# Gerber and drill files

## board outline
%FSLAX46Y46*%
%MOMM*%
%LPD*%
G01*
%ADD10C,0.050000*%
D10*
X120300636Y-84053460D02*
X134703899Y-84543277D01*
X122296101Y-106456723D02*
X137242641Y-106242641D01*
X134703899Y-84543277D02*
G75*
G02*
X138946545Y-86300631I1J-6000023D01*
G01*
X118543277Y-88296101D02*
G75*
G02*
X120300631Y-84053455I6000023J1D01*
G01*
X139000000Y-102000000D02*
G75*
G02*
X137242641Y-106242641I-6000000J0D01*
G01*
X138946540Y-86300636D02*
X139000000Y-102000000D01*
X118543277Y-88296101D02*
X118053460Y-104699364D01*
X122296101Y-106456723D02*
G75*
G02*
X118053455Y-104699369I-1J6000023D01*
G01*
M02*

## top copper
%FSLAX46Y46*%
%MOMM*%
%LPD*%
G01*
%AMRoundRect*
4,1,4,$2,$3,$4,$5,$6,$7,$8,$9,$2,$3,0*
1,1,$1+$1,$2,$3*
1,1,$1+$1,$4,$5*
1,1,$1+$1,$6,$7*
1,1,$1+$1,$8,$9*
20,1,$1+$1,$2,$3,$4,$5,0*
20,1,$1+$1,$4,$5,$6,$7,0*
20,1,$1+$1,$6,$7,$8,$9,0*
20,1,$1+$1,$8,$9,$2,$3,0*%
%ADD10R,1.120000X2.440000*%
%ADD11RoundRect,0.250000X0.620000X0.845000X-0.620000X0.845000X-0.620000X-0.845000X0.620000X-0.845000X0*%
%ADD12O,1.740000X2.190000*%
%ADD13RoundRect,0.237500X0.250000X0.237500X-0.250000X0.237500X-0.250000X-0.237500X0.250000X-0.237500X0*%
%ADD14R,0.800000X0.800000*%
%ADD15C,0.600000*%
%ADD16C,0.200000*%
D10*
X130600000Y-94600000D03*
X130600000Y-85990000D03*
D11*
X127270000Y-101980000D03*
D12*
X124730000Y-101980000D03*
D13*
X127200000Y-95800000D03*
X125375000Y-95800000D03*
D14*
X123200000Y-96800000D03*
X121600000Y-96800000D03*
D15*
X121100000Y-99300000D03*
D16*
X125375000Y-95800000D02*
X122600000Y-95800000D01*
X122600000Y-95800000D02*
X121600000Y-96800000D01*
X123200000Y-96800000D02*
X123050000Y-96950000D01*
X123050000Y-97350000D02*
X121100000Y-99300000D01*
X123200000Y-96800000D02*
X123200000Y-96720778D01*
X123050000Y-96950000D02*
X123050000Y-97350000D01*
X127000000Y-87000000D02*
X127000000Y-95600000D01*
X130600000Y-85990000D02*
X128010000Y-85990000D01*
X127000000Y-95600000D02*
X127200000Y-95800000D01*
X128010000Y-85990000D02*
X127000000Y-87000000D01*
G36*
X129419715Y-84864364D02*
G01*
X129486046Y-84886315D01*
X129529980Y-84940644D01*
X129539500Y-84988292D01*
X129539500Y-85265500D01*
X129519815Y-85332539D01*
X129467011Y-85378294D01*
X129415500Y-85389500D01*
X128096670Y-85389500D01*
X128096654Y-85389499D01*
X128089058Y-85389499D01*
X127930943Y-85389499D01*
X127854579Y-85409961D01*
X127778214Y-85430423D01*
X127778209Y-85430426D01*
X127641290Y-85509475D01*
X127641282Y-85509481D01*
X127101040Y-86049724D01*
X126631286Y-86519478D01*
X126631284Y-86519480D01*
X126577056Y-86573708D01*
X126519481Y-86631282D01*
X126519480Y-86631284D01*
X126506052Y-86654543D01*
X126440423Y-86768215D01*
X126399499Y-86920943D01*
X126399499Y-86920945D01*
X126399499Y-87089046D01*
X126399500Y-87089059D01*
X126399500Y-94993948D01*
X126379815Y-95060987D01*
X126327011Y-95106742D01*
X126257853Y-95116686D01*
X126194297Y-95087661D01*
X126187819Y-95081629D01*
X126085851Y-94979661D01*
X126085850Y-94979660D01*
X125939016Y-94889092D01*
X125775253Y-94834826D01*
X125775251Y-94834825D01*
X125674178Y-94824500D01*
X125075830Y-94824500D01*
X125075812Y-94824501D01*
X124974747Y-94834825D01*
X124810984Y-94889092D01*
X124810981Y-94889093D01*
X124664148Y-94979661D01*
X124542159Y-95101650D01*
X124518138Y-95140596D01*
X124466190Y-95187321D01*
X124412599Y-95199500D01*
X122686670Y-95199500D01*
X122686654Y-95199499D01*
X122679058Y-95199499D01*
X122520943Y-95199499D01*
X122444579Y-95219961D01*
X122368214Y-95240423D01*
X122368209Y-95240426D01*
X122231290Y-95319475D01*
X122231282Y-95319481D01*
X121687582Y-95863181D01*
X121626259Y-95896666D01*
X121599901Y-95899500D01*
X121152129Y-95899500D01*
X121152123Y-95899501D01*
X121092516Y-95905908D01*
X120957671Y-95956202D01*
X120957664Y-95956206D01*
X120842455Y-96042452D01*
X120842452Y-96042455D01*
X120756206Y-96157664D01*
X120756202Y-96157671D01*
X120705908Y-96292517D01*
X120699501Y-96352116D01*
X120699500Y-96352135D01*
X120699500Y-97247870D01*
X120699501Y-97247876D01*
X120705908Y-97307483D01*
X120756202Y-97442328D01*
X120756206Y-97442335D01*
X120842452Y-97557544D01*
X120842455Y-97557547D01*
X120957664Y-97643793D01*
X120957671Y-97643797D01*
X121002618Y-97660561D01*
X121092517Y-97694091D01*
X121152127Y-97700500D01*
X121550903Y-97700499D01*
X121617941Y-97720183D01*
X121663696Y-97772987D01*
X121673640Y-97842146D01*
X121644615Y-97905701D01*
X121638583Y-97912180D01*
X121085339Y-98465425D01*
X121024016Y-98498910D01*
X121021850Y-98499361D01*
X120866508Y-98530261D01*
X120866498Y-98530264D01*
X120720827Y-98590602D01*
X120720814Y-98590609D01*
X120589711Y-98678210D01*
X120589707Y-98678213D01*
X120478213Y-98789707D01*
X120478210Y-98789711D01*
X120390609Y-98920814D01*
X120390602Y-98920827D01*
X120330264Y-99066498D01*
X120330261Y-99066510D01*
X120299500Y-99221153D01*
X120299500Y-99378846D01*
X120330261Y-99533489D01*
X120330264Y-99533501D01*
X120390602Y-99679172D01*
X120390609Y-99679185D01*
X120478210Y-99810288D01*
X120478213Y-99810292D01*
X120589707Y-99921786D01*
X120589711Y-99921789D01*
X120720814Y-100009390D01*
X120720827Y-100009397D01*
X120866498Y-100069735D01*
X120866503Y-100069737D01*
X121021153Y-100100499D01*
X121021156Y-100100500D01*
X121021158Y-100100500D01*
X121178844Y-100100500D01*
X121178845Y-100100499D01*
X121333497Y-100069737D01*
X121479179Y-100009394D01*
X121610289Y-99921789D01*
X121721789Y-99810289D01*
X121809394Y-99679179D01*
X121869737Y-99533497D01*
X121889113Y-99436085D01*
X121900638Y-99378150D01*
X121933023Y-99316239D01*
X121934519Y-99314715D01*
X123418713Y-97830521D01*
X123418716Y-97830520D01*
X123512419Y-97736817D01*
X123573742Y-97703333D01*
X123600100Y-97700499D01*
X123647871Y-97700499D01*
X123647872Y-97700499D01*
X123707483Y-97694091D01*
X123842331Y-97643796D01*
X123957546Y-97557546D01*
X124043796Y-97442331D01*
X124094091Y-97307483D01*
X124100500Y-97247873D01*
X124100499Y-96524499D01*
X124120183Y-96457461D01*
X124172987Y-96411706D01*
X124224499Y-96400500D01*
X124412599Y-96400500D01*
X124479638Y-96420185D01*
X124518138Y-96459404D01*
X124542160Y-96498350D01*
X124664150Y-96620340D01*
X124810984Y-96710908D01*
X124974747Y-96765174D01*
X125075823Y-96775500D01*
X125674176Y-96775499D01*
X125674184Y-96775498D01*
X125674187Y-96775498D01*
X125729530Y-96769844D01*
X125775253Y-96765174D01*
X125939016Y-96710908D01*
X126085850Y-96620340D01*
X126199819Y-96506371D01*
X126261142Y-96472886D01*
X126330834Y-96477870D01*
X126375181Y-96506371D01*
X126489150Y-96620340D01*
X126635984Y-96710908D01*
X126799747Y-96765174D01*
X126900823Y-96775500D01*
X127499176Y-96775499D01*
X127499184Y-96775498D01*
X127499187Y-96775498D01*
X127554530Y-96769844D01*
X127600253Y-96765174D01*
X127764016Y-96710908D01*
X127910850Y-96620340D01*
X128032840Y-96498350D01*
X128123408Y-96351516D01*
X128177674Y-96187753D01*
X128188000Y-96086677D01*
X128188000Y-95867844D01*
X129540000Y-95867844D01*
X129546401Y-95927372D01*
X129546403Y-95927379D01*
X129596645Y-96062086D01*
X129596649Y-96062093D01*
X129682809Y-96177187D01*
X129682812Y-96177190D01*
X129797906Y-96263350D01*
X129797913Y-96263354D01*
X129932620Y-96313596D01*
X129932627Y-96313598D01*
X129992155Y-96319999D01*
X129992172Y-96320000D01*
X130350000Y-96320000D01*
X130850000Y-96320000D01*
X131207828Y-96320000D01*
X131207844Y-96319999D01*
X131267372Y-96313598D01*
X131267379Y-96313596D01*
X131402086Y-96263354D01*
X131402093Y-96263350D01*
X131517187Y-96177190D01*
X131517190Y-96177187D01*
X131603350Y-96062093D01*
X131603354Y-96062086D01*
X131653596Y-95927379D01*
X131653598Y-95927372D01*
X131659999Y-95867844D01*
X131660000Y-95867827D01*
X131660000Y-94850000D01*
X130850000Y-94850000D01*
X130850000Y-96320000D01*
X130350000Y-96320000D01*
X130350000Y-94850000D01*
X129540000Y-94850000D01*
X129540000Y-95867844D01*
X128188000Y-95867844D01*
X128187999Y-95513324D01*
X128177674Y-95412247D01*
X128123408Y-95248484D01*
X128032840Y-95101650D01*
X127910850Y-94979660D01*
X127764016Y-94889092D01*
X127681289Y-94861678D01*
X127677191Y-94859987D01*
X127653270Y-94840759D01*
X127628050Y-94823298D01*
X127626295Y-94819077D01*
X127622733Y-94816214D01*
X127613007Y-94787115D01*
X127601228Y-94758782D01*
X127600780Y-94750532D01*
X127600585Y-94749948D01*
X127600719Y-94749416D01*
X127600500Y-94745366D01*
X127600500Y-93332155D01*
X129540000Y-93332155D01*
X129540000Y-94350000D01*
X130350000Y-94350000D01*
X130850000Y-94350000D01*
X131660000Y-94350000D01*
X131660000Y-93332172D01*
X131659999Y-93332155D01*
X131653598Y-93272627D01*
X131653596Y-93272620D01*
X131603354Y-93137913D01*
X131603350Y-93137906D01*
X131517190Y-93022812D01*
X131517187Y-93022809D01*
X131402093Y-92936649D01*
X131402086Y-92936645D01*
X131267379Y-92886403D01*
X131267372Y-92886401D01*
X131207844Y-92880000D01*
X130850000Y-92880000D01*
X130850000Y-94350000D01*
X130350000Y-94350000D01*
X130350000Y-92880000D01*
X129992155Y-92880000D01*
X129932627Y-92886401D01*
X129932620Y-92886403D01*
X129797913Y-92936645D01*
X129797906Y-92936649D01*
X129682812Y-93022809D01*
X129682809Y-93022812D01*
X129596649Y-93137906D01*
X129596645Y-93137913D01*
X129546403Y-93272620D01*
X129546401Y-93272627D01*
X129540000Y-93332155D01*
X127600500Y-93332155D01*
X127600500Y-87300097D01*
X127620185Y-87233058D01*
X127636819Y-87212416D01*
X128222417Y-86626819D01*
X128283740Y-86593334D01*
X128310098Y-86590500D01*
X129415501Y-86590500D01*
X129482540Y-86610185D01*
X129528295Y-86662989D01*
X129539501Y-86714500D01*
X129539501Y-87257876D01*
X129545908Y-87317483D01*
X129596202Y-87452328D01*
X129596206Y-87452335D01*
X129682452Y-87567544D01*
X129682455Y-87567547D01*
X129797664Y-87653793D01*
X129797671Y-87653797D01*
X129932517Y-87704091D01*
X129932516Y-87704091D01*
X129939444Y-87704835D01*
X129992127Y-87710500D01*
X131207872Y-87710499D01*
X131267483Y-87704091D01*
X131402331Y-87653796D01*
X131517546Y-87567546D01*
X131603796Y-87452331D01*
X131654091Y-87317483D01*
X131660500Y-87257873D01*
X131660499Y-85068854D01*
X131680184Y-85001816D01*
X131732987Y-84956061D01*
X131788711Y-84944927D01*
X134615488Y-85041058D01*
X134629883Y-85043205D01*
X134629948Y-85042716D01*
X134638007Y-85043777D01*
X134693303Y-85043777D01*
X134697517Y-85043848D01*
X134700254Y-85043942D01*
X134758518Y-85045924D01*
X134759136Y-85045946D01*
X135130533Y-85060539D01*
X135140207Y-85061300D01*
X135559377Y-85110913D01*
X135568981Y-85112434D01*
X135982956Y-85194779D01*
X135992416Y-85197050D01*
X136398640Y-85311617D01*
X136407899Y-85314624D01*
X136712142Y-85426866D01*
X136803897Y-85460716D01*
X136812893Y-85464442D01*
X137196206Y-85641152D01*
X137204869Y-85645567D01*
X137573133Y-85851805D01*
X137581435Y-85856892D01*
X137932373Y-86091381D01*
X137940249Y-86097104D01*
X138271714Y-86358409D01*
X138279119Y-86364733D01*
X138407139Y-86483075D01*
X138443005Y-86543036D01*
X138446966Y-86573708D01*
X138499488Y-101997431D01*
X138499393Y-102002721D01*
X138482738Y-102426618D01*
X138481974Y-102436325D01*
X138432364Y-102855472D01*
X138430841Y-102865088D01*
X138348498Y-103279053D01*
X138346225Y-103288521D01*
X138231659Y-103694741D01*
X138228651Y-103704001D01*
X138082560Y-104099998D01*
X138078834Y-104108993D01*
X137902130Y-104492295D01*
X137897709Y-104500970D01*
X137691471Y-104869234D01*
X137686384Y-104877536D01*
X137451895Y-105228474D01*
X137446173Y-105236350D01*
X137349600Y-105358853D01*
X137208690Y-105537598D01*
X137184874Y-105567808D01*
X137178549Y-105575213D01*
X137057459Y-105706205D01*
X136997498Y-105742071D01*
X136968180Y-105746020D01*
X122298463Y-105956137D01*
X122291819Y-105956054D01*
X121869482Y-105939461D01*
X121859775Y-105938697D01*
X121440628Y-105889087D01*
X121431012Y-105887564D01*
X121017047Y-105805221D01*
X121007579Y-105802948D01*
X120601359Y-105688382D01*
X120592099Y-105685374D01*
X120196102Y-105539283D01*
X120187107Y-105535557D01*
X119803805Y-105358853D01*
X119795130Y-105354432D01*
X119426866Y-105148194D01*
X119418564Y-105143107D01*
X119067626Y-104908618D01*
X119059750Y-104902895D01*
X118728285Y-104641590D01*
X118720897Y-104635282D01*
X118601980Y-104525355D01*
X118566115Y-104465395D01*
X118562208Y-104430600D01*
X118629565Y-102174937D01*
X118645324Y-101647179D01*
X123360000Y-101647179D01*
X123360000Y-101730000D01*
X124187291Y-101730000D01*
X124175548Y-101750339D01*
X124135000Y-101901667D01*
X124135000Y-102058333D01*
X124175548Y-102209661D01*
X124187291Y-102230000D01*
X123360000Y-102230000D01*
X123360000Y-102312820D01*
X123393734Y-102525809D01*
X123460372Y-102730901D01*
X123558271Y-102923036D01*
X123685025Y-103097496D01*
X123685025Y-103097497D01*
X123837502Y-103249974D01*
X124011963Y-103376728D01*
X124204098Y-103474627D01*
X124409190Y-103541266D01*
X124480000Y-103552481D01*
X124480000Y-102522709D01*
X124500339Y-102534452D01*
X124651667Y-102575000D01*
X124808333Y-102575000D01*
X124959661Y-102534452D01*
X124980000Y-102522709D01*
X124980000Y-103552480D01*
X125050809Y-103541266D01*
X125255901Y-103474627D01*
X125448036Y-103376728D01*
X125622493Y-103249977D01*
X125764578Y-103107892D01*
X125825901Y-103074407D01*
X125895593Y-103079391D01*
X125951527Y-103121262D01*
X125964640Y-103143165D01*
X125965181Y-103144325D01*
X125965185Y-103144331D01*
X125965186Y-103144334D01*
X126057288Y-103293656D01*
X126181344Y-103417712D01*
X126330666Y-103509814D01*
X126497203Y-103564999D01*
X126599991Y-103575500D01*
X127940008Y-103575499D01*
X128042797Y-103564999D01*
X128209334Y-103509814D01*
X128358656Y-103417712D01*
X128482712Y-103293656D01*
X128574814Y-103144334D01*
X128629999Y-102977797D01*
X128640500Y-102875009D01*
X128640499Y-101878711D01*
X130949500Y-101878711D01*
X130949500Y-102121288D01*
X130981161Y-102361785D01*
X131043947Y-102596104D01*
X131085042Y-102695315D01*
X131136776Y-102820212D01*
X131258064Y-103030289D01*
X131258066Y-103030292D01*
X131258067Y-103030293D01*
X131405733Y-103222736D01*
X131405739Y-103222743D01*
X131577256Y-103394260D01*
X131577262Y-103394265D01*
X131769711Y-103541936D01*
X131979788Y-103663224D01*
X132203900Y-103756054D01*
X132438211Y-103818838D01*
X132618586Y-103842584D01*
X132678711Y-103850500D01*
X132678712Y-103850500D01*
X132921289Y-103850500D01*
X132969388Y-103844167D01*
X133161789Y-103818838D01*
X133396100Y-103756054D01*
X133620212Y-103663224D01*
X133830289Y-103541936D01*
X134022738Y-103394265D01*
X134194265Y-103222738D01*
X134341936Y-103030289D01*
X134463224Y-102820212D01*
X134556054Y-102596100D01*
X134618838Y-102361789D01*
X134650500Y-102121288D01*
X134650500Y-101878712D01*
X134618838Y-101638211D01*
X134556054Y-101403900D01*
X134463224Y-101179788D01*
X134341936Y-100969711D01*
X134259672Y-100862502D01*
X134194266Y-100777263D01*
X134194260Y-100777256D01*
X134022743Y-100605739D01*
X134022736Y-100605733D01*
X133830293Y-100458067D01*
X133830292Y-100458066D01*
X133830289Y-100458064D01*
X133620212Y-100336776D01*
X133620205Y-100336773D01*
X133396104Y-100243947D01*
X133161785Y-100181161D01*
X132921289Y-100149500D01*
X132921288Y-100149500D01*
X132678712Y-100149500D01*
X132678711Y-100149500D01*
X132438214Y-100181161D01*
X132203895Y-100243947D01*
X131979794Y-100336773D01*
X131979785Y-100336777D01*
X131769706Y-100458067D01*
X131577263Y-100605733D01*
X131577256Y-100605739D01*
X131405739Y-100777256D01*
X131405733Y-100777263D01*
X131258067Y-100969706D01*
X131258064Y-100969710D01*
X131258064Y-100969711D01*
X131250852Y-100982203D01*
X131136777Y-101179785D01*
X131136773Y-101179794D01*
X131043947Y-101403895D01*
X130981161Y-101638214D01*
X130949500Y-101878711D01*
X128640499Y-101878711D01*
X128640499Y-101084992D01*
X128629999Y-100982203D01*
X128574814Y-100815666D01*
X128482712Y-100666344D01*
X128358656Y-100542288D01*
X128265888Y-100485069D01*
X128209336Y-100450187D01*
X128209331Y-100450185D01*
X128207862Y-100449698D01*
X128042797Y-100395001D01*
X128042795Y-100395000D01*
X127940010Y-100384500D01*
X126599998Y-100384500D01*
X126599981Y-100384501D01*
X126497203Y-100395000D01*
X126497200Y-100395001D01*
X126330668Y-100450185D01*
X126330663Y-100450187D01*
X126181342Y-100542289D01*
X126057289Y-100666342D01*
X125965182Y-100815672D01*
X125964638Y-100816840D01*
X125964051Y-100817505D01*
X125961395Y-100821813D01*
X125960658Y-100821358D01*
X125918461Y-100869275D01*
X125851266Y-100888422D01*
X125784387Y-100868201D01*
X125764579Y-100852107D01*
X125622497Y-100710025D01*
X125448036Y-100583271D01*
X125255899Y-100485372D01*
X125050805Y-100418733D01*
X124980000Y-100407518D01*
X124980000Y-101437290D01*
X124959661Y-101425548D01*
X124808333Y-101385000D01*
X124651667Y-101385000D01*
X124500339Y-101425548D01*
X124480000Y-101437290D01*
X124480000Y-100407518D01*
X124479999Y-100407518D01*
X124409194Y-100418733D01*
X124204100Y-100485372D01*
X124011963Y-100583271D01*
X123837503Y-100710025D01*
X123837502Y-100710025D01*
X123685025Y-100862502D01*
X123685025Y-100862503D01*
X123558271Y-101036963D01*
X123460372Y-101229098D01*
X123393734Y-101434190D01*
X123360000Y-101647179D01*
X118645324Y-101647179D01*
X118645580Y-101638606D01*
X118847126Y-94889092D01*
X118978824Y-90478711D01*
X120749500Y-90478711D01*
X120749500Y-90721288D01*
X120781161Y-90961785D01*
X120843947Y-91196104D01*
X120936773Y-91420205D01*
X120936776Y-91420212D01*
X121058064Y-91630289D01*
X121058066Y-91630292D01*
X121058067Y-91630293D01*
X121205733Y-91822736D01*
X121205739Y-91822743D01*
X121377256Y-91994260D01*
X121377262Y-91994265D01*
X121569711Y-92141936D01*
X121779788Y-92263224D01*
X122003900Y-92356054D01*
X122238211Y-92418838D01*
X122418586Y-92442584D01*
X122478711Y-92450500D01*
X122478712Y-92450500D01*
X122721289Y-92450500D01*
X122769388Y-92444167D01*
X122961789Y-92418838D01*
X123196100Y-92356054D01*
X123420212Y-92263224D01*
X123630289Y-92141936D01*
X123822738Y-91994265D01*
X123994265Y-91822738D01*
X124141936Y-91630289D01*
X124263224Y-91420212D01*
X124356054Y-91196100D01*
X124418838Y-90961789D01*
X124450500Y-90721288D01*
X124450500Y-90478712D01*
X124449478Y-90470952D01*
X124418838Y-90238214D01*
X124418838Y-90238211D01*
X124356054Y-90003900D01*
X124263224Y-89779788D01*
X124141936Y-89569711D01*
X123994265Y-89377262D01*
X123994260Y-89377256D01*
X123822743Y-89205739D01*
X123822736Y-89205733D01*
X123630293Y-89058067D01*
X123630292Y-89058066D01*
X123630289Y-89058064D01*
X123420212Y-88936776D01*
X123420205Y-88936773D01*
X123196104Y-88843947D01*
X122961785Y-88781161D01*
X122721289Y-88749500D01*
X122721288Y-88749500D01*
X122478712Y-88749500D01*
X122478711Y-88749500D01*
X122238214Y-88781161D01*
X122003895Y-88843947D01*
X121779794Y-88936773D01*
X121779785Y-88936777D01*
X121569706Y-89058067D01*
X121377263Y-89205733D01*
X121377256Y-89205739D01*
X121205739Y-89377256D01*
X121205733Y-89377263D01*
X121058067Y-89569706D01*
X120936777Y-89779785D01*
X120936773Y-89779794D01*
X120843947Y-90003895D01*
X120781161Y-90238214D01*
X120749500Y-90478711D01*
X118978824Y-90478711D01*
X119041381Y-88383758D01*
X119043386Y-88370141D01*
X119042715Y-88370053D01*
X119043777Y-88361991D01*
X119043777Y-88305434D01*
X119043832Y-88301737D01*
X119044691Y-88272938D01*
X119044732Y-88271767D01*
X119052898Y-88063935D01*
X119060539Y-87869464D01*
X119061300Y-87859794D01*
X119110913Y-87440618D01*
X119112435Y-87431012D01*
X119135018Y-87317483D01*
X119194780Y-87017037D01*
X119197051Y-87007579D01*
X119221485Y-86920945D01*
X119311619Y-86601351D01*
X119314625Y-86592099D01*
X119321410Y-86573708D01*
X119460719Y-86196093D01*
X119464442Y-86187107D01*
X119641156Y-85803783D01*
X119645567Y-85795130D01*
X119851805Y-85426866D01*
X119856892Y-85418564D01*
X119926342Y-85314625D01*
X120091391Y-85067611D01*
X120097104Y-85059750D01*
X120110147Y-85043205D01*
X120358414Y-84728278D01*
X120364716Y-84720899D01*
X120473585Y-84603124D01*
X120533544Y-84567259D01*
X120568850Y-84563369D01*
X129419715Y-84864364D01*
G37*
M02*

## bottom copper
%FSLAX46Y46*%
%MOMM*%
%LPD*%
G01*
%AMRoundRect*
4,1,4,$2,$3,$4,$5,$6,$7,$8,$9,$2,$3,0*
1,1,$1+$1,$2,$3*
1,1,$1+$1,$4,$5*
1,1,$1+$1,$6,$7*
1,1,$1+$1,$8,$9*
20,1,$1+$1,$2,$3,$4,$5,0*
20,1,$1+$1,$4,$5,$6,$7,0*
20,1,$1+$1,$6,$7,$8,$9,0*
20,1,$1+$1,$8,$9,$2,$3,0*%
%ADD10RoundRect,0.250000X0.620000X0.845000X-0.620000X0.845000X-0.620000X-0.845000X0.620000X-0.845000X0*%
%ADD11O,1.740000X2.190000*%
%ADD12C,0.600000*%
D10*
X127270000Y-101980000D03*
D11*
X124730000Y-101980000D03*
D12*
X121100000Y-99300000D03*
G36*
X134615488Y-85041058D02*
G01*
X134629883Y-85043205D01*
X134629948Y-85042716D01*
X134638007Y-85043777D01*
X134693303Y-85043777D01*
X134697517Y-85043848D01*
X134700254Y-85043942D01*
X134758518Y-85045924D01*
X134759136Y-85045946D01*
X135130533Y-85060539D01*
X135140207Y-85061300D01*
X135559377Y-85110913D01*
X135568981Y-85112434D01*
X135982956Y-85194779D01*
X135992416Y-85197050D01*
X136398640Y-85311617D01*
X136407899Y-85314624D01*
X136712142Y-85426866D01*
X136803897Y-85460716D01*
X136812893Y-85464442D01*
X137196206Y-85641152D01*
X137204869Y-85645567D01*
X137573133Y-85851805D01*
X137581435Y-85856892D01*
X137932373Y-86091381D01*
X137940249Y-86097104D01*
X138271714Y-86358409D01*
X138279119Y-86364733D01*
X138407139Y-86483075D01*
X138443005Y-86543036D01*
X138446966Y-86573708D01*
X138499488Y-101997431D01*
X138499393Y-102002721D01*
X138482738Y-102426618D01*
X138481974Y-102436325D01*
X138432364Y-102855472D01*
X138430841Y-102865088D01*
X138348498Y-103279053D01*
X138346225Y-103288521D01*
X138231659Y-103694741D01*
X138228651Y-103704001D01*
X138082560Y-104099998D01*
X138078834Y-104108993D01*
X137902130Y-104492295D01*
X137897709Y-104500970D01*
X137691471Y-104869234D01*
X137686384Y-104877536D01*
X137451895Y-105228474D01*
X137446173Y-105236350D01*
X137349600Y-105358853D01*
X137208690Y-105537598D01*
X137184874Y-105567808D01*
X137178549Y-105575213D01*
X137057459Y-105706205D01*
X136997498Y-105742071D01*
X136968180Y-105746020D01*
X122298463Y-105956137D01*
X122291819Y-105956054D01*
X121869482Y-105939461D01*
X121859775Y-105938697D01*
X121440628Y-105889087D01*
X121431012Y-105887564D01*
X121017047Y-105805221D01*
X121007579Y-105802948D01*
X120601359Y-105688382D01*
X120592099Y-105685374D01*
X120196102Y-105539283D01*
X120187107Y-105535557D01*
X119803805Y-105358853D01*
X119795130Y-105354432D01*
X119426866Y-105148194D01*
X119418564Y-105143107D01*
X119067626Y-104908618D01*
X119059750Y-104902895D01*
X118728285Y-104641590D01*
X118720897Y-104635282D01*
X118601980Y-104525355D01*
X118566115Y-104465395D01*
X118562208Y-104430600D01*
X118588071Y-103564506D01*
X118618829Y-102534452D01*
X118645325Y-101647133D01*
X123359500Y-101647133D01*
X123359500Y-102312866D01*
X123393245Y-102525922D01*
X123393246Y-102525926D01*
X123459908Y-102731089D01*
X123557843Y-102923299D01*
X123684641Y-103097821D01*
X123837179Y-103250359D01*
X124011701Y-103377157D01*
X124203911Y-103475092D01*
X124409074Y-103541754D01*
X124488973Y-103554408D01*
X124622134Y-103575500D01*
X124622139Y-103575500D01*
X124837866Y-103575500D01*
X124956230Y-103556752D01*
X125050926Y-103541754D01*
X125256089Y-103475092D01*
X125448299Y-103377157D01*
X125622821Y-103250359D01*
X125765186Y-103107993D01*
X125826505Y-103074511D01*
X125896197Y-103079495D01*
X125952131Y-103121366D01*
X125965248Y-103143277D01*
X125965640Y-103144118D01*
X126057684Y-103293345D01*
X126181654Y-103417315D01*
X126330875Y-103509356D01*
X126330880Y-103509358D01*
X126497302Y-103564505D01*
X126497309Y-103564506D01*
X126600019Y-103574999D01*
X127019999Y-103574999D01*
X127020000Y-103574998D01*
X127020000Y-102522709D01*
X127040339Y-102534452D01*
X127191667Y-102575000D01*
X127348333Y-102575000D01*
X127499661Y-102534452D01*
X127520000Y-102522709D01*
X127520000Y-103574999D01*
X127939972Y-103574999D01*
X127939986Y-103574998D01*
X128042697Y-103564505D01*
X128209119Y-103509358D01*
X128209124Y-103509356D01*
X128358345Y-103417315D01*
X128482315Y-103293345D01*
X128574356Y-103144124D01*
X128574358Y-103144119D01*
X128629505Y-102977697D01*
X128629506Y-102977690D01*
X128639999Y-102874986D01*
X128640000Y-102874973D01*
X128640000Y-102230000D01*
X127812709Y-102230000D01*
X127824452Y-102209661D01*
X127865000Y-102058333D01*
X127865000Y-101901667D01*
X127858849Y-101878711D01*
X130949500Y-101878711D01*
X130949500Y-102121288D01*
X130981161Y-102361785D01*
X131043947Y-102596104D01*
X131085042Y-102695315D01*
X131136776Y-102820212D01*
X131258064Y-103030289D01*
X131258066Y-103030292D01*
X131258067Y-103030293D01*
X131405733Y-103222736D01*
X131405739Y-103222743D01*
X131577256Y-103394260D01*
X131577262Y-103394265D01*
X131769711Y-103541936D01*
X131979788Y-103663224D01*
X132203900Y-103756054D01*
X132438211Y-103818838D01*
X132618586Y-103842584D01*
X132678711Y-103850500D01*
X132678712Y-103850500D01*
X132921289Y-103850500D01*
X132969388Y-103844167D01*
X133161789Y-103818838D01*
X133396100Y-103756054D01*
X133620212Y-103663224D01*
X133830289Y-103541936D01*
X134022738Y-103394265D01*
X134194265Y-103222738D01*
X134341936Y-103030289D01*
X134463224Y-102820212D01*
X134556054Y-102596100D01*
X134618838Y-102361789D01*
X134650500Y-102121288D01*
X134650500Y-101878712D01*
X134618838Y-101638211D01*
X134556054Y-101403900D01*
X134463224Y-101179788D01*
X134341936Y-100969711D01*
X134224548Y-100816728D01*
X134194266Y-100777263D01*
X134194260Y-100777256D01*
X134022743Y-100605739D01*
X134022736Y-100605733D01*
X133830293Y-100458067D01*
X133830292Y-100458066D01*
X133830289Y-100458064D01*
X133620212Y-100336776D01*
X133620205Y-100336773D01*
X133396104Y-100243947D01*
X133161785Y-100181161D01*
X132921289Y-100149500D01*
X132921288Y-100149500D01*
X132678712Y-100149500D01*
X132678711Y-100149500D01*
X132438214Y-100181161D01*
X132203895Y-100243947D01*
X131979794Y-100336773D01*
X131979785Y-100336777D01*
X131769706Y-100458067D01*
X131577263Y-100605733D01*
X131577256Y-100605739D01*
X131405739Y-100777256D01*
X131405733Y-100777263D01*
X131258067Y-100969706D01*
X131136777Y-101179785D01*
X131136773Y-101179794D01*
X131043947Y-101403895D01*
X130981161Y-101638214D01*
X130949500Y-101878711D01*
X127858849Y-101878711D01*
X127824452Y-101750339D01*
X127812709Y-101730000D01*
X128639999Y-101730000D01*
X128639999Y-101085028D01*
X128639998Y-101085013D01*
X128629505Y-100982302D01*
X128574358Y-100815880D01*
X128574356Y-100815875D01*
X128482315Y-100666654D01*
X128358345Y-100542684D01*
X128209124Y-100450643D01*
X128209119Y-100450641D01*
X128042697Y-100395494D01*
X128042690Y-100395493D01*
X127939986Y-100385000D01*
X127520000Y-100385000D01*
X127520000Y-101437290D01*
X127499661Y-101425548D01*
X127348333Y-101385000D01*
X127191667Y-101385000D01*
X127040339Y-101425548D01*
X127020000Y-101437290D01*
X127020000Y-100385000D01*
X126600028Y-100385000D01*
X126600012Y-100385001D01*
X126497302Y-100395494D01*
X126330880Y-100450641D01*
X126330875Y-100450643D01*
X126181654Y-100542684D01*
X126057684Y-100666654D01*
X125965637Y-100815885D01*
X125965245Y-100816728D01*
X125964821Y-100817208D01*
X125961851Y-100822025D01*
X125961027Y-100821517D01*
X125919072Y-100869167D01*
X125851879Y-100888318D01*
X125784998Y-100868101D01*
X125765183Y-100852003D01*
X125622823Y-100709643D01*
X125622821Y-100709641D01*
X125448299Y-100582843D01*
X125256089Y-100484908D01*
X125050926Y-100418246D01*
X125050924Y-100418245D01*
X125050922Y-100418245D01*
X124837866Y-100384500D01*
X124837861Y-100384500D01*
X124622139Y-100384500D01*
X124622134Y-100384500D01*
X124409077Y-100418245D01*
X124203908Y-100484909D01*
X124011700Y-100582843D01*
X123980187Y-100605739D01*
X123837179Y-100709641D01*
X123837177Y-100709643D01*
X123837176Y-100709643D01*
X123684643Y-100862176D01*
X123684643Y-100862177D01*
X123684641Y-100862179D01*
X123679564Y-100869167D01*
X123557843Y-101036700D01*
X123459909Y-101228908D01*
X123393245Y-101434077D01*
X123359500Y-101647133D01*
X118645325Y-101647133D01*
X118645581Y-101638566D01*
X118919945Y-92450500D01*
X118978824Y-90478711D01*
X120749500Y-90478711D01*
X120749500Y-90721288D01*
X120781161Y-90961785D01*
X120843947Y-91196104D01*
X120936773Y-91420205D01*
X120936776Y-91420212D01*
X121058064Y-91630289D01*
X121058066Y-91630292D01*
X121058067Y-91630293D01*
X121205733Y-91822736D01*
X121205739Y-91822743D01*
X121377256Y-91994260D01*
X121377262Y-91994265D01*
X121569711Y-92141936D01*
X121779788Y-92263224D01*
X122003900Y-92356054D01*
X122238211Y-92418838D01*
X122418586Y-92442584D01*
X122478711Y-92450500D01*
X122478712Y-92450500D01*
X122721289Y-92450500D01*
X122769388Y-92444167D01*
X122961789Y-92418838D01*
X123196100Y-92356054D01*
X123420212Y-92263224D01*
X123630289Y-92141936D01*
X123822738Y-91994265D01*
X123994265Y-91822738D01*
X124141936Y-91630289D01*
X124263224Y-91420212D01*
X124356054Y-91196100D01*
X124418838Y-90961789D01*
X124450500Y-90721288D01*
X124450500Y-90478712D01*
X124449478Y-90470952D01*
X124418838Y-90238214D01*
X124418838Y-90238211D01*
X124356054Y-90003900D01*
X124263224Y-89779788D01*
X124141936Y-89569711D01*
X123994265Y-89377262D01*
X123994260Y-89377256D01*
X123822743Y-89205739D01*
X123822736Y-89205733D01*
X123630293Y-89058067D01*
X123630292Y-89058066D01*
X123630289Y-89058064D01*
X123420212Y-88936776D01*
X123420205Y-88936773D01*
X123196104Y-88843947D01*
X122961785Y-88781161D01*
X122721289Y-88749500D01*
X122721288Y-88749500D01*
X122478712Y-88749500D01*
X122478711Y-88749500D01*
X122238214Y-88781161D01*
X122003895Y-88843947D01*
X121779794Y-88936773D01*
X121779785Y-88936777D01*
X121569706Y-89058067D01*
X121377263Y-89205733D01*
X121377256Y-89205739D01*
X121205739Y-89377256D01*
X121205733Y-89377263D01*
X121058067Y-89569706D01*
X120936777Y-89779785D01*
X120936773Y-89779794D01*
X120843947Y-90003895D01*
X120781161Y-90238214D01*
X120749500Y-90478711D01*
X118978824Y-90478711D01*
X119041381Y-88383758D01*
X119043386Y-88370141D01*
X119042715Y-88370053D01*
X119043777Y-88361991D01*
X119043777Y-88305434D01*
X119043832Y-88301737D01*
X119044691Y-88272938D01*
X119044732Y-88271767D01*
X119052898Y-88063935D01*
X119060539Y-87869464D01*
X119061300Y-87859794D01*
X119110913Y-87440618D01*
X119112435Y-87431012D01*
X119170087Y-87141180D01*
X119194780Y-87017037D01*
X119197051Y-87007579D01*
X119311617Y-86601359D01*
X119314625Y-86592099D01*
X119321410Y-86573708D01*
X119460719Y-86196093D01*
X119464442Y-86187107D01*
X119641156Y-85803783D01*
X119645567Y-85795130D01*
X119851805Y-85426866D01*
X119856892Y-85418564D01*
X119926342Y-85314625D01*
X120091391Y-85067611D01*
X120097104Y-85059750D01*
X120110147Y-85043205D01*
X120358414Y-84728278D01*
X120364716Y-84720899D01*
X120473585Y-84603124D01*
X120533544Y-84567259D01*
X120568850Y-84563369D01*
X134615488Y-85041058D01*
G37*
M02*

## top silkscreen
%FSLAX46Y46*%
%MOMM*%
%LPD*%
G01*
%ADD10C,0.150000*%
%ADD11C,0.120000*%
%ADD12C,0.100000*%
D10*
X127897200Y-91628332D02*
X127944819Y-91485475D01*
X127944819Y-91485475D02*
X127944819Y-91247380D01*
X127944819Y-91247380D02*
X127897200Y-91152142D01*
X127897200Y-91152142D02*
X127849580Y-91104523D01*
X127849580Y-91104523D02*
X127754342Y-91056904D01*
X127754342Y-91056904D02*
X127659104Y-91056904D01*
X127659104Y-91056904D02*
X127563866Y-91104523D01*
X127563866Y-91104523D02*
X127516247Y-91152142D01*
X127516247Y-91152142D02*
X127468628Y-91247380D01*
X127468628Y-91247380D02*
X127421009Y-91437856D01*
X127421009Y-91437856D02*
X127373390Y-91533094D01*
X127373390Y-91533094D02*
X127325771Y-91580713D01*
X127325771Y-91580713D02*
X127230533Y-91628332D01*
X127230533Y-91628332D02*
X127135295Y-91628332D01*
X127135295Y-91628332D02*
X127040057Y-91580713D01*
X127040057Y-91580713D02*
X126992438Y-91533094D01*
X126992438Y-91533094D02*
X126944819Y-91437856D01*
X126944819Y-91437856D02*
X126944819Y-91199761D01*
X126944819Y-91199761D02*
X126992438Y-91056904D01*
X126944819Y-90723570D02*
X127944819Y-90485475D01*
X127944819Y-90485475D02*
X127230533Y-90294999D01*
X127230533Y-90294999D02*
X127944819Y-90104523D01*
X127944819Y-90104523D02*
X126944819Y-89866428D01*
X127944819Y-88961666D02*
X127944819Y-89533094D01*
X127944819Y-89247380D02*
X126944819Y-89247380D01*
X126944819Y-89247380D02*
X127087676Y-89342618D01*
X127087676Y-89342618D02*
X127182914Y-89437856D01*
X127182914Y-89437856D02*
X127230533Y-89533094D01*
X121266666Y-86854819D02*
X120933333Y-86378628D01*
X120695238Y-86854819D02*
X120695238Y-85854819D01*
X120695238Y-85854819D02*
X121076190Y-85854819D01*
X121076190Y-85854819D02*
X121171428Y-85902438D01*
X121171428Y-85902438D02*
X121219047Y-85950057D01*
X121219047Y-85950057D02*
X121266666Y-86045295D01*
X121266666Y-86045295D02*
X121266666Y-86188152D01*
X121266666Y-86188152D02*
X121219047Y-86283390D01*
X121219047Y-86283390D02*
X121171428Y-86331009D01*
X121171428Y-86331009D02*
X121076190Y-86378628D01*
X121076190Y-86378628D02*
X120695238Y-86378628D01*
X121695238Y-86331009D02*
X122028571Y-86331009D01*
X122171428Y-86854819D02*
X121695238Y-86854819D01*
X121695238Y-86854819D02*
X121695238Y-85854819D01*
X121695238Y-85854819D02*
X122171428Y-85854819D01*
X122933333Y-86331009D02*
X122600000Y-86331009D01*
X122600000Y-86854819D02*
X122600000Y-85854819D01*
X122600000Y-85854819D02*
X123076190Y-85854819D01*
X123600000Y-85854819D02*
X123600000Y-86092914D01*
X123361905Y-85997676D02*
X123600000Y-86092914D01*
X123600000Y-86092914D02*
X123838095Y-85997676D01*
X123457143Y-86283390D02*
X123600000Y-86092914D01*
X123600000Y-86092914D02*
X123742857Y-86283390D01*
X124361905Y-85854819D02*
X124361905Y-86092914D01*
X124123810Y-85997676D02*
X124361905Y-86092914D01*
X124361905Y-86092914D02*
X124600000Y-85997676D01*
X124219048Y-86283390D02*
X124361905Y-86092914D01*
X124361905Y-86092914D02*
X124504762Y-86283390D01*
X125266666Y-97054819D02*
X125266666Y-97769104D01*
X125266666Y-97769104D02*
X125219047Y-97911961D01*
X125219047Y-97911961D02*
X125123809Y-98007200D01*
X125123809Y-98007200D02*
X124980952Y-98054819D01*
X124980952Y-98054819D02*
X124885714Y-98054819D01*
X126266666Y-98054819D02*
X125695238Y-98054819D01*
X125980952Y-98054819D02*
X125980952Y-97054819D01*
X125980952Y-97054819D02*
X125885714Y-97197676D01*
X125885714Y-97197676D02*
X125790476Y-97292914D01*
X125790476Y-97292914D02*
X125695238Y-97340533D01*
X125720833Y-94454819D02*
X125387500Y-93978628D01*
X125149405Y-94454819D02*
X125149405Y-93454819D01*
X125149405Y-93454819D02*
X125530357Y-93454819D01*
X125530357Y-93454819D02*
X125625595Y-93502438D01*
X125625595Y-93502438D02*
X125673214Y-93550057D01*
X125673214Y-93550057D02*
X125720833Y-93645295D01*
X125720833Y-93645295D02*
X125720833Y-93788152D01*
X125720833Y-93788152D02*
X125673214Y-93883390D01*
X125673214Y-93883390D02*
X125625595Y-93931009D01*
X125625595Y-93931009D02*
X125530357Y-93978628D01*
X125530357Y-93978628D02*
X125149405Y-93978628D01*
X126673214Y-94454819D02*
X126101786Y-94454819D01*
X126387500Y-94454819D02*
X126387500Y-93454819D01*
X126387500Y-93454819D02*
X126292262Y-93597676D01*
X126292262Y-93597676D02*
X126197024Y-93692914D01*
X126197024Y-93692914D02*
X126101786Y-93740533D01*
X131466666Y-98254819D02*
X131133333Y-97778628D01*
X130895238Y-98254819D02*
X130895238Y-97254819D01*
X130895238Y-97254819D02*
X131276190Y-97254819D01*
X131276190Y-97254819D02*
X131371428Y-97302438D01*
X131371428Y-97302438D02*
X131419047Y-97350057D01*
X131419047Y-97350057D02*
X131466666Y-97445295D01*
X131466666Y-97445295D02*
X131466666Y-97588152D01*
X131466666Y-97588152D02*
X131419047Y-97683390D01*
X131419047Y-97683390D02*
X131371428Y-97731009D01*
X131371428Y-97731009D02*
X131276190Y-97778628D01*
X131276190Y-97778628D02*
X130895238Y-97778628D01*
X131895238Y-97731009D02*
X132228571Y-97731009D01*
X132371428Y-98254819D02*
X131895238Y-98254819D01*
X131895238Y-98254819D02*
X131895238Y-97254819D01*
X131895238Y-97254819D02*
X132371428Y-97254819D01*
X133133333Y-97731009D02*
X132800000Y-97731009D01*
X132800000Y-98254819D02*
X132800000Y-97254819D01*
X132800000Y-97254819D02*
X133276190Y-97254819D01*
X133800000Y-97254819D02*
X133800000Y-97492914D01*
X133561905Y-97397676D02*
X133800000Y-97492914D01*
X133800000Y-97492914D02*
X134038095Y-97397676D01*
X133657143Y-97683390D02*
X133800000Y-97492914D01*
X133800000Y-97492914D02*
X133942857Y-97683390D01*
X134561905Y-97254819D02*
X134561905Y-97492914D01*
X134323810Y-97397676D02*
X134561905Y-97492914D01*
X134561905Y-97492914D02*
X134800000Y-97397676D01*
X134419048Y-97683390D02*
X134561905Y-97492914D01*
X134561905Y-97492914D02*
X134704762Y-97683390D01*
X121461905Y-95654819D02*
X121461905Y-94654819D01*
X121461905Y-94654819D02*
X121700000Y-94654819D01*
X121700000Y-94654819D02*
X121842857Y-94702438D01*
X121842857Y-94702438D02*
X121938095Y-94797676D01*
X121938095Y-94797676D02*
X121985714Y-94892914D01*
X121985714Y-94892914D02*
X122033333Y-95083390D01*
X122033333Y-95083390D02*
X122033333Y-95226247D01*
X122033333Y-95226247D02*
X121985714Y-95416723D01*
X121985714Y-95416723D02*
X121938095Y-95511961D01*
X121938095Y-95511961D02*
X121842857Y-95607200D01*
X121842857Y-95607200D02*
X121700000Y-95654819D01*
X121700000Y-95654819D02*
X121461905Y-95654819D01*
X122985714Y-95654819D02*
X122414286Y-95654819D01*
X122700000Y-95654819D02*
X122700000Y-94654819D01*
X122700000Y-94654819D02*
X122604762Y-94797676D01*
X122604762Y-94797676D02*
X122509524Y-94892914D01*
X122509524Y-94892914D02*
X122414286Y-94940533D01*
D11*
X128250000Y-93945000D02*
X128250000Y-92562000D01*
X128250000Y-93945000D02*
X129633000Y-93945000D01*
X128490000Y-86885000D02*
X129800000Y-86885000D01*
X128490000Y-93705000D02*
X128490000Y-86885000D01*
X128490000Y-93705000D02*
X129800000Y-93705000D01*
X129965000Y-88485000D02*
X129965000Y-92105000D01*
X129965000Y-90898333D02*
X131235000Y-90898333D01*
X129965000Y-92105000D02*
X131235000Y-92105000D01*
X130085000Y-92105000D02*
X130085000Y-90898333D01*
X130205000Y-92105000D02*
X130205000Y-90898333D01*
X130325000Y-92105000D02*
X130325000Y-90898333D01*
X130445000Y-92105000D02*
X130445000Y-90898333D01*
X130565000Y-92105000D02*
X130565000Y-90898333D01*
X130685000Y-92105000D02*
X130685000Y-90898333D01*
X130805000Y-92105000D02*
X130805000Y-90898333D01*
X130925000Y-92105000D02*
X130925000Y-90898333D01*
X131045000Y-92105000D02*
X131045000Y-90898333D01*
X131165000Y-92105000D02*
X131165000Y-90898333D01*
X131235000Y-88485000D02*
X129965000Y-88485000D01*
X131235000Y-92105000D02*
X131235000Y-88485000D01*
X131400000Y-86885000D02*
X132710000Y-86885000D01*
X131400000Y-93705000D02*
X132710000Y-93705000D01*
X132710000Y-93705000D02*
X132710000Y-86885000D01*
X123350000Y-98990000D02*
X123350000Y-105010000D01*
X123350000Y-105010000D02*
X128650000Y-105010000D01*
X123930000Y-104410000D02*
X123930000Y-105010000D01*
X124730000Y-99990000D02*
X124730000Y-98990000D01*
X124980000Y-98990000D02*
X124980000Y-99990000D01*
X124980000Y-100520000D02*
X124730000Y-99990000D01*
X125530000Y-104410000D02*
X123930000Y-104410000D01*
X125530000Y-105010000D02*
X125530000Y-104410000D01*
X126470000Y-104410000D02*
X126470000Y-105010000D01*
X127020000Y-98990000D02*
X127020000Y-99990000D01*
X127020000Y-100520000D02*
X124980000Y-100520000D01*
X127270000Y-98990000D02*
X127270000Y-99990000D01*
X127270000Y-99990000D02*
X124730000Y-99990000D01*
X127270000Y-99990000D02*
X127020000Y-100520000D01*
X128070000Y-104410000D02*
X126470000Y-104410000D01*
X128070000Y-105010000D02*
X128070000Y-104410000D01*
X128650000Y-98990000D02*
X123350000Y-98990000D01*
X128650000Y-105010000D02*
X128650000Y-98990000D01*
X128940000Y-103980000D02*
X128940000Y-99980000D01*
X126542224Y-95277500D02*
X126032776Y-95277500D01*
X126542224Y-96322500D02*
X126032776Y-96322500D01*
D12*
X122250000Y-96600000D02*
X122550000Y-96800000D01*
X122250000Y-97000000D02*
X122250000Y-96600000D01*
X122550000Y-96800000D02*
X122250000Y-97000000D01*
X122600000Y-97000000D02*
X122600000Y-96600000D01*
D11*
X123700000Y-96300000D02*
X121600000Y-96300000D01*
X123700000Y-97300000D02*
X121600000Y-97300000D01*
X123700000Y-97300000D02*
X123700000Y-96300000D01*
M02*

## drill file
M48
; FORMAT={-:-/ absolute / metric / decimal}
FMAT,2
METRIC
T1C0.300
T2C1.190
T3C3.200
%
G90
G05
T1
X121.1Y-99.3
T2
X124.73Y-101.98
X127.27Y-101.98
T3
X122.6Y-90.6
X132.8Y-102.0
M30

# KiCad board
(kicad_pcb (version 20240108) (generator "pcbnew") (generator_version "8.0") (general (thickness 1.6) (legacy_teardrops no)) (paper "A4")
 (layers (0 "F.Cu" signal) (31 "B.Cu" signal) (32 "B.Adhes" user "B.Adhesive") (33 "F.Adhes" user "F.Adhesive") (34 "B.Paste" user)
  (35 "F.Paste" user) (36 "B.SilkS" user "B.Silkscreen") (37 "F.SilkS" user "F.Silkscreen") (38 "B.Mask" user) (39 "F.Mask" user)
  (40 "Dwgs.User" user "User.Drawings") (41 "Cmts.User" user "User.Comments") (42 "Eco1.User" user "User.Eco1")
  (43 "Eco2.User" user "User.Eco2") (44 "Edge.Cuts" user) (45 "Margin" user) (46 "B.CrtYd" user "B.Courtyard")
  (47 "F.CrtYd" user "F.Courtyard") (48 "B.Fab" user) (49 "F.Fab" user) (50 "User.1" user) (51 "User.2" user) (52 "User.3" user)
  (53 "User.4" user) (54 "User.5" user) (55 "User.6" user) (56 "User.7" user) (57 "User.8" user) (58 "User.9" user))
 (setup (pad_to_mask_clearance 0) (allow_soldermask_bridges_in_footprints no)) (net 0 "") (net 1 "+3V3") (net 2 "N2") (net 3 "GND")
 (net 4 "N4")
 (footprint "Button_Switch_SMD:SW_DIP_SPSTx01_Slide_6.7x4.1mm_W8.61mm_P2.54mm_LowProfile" (layer "F.Cu") (at 130.6 90.295 90)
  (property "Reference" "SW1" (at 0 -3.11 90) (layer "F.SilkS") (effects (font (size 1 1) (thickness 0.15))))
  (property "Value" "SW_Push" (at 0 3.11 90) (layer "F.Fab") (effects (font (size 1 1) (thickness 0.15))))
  (fp_line (start -3.65 -2.35) (end -2.267 -2.35) (stroke (width 0.12) (type solid)) (layer "F.SilkS"))
  (fp_line (start -3.65 -2.35) (end -3.65 -0.967) (stroke (width 0.12) (type solid)) (layer "F.SilkS"))
  (fp_line (start 3.41 -2.11) (end 3.41 -0.8) (stroke (width 0.12) (type solid)) (layer "F.SilkS"))
  (fp_line (start -3.41 -2.11) (end 3.41 -2.11) (stroke (width 0.12) (type solid)) (layer "F.SilkS"))
  (fp_line (start -3.41 -2.11) (end -3.41 -0.8) (stroke (width 0.12) (type solid)) (layer "F.SilkS"))
  (fp_line (start 1.81 -0.635) (end -1.81 -0.635) (stroke (width 0.12) (type solid)) (layer "F.SilkS"))
  (fp_line (start -0.603333 -0.635) (end -0.603333 0.635) (stroke (width 0.12) (type solid)) (layer "F.SilkS"))
  (fp_line (start -1.81 -0.635) (end -1.81 0.635) (stroke (width 0.12) (type solid)) (layer "F.SilkS"))
  (fp_line (start -1.81 -0.515) (end -0.603333 -0.515) (stroke (width 0.12) (type solid)) (layer "F.SilkS"))
  (fp_line (start -1.81 -0.395) (end -0.603333 -0.395) (stroke (width 0.12) (type solid)) (layer "F.SilkS"))
  (fp_line (start -1.81 -0.275) (end -0.603333 -0.275) (stroke (width 0.12) (type solid)) (layer "F.SilkS"))
  (fp_line (start -1.81 -0.155) (end -0.603333 -0.155) (stroke (width 0.12) (type solid)) (layer "F.SilkS"))
  (fp_line (start -1.81 -0.035) (end -0.603333 -0.035) (stroke (width 0.12) (type solid)) (layer "F.SilkS"))
  (fp_line (start -1.81 0.085) (end -0.603333 0.085) (stroke (width 0.12) (type solid)) (layer "F.SilkS"))
  (fp_line (start -1.81 0.205) (end -0.603333 0.205) (stroke (width 0.12) (type solid)) (layer "F.SilkS"))
  (fp_line (start -1.81 0.325) (end -0.603333 0.325) (stroke (width 0.12) (type solid)) (layer "F.SilkS"))
  (fp_line (start -1.81 0.445) (end -0.603333 0.445) (stroke (width 0.12) (type solid)) (layer "F.SilkS"))
  (fp_line (start -1.81 0.565) (end -0.603333 0.565) (stroke (width 0.12) (type solid)) (layer "F.SilkS"))
  (fp_line (start 1.81 0.635) (end 1.81 -0.635) (stroke (width 0.12) (type solid)) (layer "F.SilkS"))
  (fp_line (start -1.81 0.635) (end 1.81 0.635) (stroke (width 0.12) (type solid)) (layer "F.SilkS"))
  (fp_line (start 3.41 0.8) (end 3.41 2.11) (stroke (width 0.12) (type solid)) (layer "F.SilkS"))
  (fp_line (start -3.41 0.8) (end -3.41 2.11) (stroke (width 0.12) (type solid)) (layer "F.SilkS"))
  (fp_line (start -3.41 2.11) (end 3.41 2.11) (stroke (width 0.12) (type solid)) (layer "F.SilkS"))
  (pad "1" smd rect (at -4.305 0 90) (size 2.44 1.12) (layers "F.Cu" "F.Paste" "F.Mask") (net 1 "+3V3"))
  (pad "2" smd rect (at 4.305 0 90) (size 2.44 1.12) (layers "F.Cu" "F.Paste" "F.Mask") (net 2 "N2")))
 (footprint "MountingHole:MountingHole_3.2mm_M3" (layer "F.Cu") (at 122.6 90.6)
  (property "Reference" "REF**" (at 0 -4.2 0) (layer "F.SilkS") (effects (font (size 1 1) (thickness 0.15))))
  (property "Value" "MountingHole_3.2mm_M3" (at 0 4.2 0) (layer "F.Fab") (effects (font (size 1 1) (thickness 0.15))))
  (pad "" np_thru_hole circle (at 0 0) (size 3.2 3.2) (drill 3.2) (layers "*.Cu" "*.Mask")))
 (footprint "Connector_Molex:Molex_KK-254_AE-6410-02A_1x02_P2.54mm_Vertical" (layer "F.Cu") (at 127.27 101.98 180)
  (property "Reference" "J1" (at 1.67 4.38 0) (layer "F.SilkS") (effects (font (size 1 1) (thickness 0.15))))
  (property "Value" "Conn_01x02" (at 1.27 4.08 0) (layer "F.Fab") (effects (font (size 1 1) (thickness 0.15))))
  (fp_line (start 3.92 2.99) (end 3.92 -3.03) (stroke (width 0.12) (type solid)) (layer "F.SilkS"))
  (fp_line (start 3.92 -3.03) (end -1.38 -3.03) (stroke (width 0.12) (type solid)) (layer "F.SilkS"))
  (fp_line (start 3.34 -2.43) (end 3.34 -3.03) (stroke (width 0.12) (type solid)) (layer "F.SilkS"))
  (fp_line (start 2.54 1.99) (end 2.54 2.99) (stroke (width 0.12) (type solid)) (layer "F.SilkS"))
  (fp_line (start 2.29 2.99) (end 2.29 1.99) (stroke (width 0.12) (type solid)) (layer "F.SilkS"))
  (fp_line (start 2.29 1.46) (end 2.54 1.99) (stroke (width 0.12) (type solid)) (layer "F.SilkS"))
  (fp_line (start 1.74 -2.43) (end 3.34 -2.43) (stroke (width 0.12) (type solid)) (layer "F.SilkS"))
  (fp_line (start 1.74 -3.03) (end 1.74 -2.43) (stroke (width 0.12) (type solid)) (layer "F.SilkS"))
  (fp_line (start 0.8 -2.43) (end 0.8 -3.03) (stroke (width 0.12) (type solid)) (layer "F.SilkS"))
  (fp_line (start 0.25 2.99) (end 0.25 1.99) (stroke (width 0.12) (type solid)) (layer "F.SilkS"))
  (fp_line (start 0.25 1.46) (end 2.29 1.46) (stroke (width 0.12) (type solid)) (layer "F.SilkS"))
  (fp_line (start 0 2.99) (end 0 1.99) (stroke (width 0.12) (type solid)) (layer "F.SilkS"))
  (fp_line (start 0 1.99) (end 2.54 1.99) (stroke (width 0.12) (type solid)) (layer "F.SilkS"))
  (fp_line (start 0 1.99) (end 0.25 1.46) (stroke (width 0.12) (type solid)) (layer "F.SilkS"))
  (fp_line (start -0.8 -2.43) (end 0.8 -2.43) (stroke (width 0.12) (type solid)) (layer "F.SilkS"))
  (fp_line (start -0.8 -3.03) (end -0.8 -2.43) (stroke (width 0.12) (type solid)) (layer "F.SilkS"))
  (fp_line (start -1.38 2.99) (end 3.92 2.99) (stroke (width 0.12) (type solid)) (layer "F.SilkS"))
  (fp_line (start -1.38 -3.03) (end -1.38 2.99) (stroke (width 0.12) (type solid)) (layer "F.SilkS"))
  (fp_line (start -1.67 -2) (end -1.67 2) (stroke (width 0.12) (type solid)) (layer "F.SilkS"))
  (pad "1" thru_hole roundrect (at 0 0 180) (size 1.74 2.19) (drill 1.19) (layers "*.Cu" "*.Mask") (remove_unused_layers no)
   (roundrect_rratio 0.143678) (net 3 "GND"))
  (pad "2" thru_hole oval (at 2.54 0 180) (size 1.74 2.19) (drill 1.19) (layers "*.Cu" "*.Mask") (remove_unused_layers no) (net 1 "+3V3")))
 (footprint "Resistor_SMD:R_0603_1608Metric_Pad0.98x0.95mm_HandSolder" (layer "F.Cu") (at 126.2875 95.8 180)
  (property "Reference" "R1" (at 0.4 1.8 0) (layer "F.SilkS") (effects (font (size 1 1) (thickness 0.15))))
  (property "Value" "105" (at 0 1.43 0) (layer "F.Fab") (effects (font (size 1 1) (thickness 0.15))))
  (fp_line (start -0.254724 0.5225) (end 0.254724 0.5225) (stroke (width 0.12) (type solid)) (layer "F.SilkS"))
  (fp_line (start -0.254724 -0.5225) (end 0.254724 -0.5225) (stroke (width 0.12) (type solid)) (layer "F.SilkS"))
  (pad "1" smd roundrect (at -0.9125 0 180) (size 0.975 0.95) (layers "F.Cu" "F.Paste" "F.Mask") (roundrect_rratio 0.25) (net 2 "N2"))
  (pad "2" smd roundrect (at 0.9125 0 180) (size 0.975 0.95) (layers "F.Cu" "F.Paste" "F.Mask") (roundrect_rratio 0.25) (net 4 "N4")))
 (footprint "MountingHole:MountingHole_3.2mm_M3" (layer "F.Cu") (at 132.8 102)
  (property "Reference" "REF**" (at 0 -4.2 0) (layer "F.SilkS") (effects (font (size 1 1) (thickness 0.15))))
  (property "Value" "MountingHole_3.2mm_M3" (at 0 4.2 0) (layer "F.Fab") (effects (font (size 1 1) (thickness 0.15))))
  (pad "" np_thru_hole circle (at 0 0) (size 3.2 3.2) (drill 3.2) (layers "*.Cu" "*.Mask")))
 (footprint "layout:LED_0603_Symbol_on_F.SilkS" (layer "F.Cu") (at 122.4 96.8 180)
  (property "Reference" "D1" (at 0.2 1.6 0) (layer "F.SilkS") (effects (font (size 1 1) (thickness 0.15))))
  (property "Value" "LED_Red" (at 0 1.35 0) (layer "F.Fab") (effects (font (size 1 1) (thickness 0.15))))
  (fp_line (start 0.15 0.2) (end -0.15 0) (stroke (width 0.1) (type solid)) (layer "F.SilkS"))
  (fp_line (start 0.15 -0.2) (end 0.15 0.2) (stroke (width 0.1) (type solid)) (layer "F.SilkS"))
  (fp_line (start -0.15 0) (end 0.15 -0.2) (stroke (width 0.1) (type solid)) (layer "F.SilkS"))
  (fp_line (start -0.2 -0.2) (end -0.2 0.2) (stroke (width 0.1) (type solid)) (layer "F.SilkS"))
  (fp_line (start -1.3 0.5) (end 0.8 0.5) (stroke (width 0.12) (type solid)) (layer "F.SilkS"))
  (fp_line (start -1.3 -0.5) (end 0.8 -0.5) (stroke (width 0.12) (type solid)) (layer "F.SilkS"))
  (fp_line (start -1.3 -0.5) (end -1.3 0.5) (stroke (width 0.12) (type solid)) (layer "F.SilkS"))
  (pad "1" smd rect (at -0.8 0) (size 0.8 0.8) (layers "F.Cu" "F.Paste" "F.Mask") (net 3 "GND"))
  (pad "2" smd rect (at 0.8 0) (size 0.8 0.8) (layers "F.Cu" "F.Paste" "F.Mask") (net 4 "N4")))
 (gr_line (start 120.300636 84.05346) (end 134.703899 84.543277) (stroke (width 0.05) (type default)) (layer "Edge.Cuts"))
 (gr_line (start 122.296101 106.456723) (end 137.242641 106.242641) (stroke (width 0.05) (type default)) (layer "Edge.Cuts"))
 (gr_arc (start 134.703899 84.543277) (mid 137 85) (end 138.94654 86.300636) (stroke (width 0.05) (type default)) (layer "Edge.Cuts"))
 (gr_arc (start 118.543277 88.296101) (mid 119 86) (end 120.300636 84.05346) (stroke (width 0.05) (type default)) (layer "Edge.Cuts"))
 (gr_arc (start 139 102) (mid 138.543277 104.296101) (end 137.242641 106.242641) (stroke (width 0.05) (type default)) (layer "Edge.Cuts"))
 (gr_line (start 138.94654 86.300636) (end 139 102) (stroke (width 0.05) (type default)) (layer "Edge.Cuts"))
 (gr_line (start 118.543277 88.296101) (end 118.05346 104.699364) (stroke (width 0.05) (type default)) (layer "Edge.Cuts"))
 (gr_arc (start 122.296101 106.456723) (mid 120 106) (end 118.05346 104.699364) (stroke (width 0.05) (type default)) (layer "Edge.Cuts"))
 (segment (start 125.375 95.8) (end 122.6 95.8) (width 0.2) (layer "F.Cu") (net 4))
 (segment (start 122.6 95.8) (end 121.6 96.8) (width 0.2) (layer "F.Cu") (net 4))
 (segment (start 123.2 96.8) (end 123.05 96.95) (width 0.2) (layer "F.Cu") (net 3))
 (segment (start 123.05 97.35) (end 121.1 99.3) (width 0.2) (layer "F.Cu") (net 3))
 (segment (start 123.2 96.8) (end 123.2 96.720778) (width 0.2) (layer "F.Cu") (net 3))
 (segment (start 123.05 96.95) (end 123.05 97.35) (width 0.2) (layer "F.Cu") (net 3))
 (via (at 121.1 99.3) (size 0.6) (drill 0.3) (layers "F.Cu" "B.Cu") (free yes) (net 3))
 (segment (start 127 87) (end 127 95.6) (width 0.2) (layer "F.Cu") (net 2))
 (segment (start 130.6 85.99) (end 128.01 85.99) (width 0.2) (layer "F.Cu") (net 2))
 (segment (start 127 95.6) (end 127.2 95.8) (width 0.2) (layer "F.Cu") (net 2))
 (segment (start 128.01 85.99) (end 127 87) (width 0.2) (layer "F.Cu") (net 2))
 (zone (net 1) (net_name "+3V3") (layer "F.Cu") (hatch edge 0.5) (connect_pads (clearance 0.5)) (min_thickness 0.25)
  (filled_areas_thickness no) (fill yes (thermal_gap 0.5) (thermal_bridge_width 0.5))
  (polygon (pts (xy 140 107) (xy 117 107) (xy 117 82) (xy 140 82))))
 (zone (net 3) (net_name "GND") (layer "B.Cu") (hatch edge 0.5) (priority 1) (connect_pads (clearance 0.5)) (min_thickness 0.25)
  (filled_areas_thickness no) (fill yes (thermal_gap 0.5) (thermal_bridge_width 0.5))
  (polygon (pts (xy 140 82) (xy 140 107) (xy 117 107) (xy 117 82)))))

